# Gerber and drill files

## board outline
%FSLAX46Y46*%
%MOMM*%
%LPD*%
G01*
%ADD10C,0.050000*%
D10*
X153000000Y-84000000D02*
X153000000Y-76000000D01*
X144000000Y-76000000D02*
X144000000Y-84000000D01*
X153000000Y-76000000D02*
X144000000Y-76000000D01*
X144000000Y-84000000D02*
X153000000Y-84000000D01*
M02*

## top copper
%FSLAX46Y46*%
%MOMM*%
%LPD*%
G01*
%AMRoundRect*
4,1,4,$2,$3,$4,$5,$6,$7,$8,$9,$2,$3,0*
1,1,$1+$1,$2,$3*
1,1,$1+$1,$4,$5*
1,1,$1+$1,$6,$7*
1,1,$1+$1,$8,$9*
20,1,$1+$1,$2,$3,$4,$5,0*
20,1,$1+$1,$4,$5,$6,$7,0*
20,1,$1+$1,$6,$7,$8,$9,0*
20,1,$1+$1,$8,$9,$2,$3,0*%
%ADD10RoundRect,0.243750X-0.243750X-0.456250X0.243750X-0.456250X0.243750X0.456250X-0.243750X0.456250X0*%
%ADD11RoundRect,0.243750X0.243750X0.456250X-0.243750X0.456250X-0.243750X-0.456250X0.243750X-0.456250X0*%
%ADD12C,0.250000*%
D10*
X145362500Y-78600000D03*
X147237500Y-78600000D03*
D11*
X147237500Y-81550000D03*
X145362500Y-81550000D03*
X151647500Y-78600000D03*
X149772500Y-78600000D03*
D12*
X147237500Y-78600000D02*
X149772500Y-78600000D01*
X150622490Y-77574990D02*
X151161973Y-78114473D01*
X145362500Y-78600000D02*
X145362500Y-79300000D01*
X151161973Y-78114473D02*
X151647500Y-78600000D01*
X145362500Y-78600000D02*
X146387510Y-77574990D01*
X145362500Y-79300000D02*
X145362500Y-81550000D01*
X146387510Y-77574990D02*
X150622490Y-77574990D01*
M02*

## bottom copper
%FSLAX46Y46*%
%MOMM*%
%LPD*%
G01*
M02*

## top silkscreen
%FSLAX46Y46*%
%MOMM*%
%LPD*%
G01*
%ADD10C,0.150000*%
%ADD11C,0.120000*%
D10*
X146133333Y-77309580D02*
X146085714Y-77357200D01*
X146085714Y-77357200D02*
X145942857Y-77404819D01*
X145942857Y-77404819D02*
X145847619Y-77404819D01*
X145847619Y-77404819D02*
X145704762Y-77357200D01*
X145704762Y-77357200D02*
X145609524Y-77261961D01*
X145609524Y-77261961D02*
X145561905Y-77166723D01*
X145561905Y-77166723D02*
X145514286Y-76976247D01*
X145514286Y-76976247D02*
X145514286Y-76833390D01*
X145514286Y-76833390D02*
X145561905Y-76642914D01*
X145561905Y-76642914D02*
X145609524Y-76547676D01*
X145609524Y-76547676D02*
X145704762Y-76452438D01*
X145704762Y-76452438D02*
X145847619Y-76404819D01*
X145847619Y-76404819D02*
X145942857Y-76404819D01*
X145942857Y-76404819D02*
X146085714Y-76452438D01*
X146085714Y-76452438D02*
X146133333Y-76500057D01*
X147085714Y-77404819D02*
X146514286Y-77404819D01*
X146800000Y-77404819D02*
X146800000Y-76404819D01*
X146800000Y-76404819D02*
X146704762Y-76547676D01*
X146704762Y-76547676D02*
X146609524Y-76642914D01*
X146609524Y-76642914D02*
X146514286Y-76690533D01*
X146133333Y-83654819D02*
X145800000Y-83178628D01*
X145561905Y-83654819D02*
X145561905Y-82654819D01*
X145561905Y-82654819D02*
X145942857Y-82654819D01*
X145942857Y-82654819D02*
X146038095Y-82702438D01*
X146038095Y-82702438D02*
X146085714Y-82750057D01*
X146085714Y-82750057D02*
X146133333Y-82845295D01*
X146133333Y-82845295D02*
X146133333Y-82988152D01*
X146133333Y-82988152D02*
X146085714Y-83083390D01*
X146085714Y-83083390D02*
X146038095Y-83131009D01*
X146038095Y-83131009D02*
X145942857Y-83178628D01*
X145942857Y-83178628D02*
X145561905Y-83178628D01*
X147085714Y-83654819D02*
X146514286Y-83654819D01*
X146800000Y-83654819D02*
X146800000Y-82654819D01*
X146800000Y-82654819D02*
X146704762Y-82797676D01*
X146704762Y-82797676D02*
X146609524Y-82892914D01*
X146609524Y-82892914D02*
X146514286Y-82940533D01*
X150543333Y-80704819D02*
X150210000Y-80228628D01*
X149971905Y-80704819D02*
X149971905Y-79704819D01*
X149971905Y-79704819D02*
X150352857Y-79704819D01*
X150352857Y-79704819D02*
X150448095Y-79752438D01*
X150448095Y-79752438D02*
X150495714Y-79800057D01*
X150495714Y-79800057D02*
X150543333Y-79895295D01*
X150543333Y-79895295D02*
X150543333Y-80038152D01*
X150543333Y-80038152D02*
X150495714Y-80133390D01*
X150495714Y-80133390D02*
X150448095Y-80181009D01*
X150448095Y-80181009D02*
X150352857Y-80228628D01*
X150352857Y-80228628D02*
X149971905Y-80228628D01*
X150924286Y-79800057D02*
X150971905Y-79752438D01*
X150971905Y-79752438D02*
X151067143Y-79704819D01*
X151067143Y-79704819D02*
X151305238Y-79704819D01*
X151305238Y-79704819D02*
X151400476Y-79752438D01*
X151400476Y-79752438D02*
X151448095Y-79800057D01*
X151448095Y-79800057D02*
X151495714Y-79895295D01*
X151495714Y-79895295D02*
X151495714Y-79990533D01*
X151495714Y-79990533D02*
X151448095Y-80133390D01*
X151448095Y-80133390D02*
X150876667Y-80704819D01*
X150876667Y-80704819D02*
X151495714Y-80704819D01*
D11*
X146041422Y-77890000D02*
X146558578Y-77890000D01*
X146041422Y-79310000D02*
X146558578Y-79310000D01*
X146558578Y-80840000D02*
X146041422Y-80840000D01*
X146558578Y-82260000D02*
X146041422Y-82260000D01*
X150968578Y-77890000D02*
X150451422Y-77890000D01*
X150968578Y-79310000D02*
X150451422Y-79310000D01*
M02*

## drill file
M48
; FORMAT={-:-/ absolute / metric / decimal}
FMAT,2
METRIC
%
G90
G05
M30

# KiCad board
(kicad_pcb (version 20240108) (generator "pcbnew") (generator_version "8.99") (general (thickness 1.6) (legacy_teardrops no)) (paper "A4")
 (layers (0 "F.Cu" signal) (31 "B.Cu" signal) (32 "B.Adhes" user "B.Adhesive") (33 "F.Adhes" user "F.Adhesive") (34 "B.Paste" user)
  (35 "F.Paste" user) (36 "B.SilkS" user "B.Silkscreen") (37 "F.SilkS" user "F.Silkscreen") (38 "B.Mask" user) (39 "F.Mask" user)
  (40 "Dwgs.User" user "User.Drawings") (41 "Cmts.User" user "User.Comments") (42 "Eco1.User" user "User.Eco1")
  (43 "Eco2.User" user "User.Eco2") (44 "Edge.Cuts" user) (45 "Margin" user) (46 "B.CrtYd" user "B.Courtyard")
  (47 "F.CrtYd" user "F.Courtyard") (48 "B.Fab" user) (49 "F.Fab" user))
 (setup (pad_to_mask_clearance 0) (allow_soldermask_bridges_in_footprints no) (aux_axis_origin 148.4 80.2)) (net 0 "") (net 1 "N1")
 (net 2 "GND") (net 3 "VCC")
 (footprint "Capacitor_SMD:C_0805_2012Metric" (layer "F.Cu") (at 146.3 78.6)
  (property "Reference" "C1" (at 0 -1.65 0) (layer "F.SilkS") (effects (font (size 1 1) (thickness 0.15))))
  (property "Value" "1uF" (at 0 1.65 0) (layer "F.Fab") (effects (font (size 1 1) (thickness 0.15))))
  (fp_line (start -0.258578 -0.71) (end 0.258578 -0.71) (stroke (width 0.12) (type solid)) (layer "F.SilkS"))
  (fp_line (start -0.258578 0.71) (end 0.258578 0.71) (stroke (width 0.12) (type solid)) (layer "F.SilkS"))
  (pad "1" smd roundrect (at -0.9375 0) (size 0.975 1.4) (layers "F.Cu" "F.Paste" "F.Mask") (roundrect_rratio 0.25) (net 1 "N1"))
  (pad "2" smd roundrect (at 0.9375 0) (size 0.975 1.4) (layers "F.Cu" "F.Paste" "F.Mask") (roundrect_rratio 0.25) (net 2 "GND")))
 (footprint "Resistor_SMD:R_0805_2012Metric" (layer "F.Cu") (at 146.3 81.55 180)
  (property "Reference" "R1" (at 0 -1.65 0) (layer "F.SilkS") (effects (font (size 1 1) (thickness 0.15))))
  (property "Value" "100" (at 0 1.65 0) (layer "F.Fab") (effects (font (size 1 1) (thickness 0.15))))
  (fp_line (start -0.258578 0.71) (end 0.258578 0.71) (stroke (width 0.12) (type solid)) (layer "F.SilkS"))
  (fp_line (start -0.258578 -0.71) (end 0.258578 -0.71) (stroke (width 0.12) (type solid)) (layer "F.SilkS"))
  (pad "1" smd roundrect (at -0.9375 0 180) (size 0.975 1.4) (layers "F.Cu" "F.Paste" "F.Mask") (roundrect_rratio 0.25) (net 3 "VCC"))
  (pad "2" smd roundrect (at 0.9375 0 180) (size 0.975 1.4) (layers "F.Cu" "F.Paste" "F.Mask") (roundrect_rratio 0.25) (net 1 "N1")))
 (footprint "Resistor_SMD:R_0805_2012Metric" (layer "F.Cu") (at 150.71 78.6 180)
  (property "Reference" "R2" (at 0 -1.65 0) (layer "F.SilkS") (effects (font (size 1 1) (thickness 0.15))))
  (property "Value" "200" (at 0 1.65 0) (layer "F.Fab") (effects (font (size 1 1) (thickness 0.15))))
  (fp_line (start -0.258578 0.71) (end 0.258578 0.71) (stroke (width 0.12) (type solid)) (layer "F.SilkS"))
  (fp_line (start -0.258578 -0.71) (end 0.258578 -0.71) (stroke (width 0.12) (type solid)) (layer "F.SilkS"))
  (pad "1" smd roundrect (at -0.9375 0 180) (size 0.975 1.4) (layers "F.Cu" "F.Paste" "F.Mask") (roundrect_rratio 0.25) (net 1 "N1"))
  (pad "2" smd roundrect (at 0.9375 0 180) (size 0.975 1.4) (layers "F.Cu" "F.Paste" "F.Mask") (roundrect_rratio 0.25) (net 2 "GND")))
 (gr_line (start 153 84) (end 153 76) (stroke (width 0.05) (type solid)) (layer "Edge.Cuts"))
 (gr_line (start 144 76) (end 144 84) (stroke (width 0.05) (type solid)) (layer "Edge.Cuts"))
 (gr_line (start 153 76) (end 144 76) (stroke (width 0.05) (type solid)) (layer "Edge.Cuts"))
 (gr_line (start 144 84) (end 153 84) (stroke (width 0.05) (type solid)) (layer "Edge.Cuts"))
 (segment (start 147.2375 78.6) (end 149.7725 78.6) (width 0.25) (layer "F.Cu") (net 2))
 (segment (start 150.62249 77.57499) (end 151.161973 78.114473) (width 0.25) (layer "F.Cu") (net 1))
 (segment (start 145.3625 78.6) (end 145.3625 79.3) (width 0.25) (layer "F.Cu") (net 1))
 (segment (start 151.161973 78.114473) (end 151.6475 78.6) (width 0.25) (layer "F.Cu") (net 1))
 (segment (start 145.3625 78.6) (end 146.38751 77.57499) (width 0.25) (layer "F.Cu") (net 1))
 (segment (start 145.3625 79.3) (end 145.3625 81.55) (width 0.25) (layer "F.Cu") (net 1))
 (segment (start 146.38751 77.57499) (end 150.62249 77.57499) (width 0.25) (layer "F.Cu") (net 1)))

